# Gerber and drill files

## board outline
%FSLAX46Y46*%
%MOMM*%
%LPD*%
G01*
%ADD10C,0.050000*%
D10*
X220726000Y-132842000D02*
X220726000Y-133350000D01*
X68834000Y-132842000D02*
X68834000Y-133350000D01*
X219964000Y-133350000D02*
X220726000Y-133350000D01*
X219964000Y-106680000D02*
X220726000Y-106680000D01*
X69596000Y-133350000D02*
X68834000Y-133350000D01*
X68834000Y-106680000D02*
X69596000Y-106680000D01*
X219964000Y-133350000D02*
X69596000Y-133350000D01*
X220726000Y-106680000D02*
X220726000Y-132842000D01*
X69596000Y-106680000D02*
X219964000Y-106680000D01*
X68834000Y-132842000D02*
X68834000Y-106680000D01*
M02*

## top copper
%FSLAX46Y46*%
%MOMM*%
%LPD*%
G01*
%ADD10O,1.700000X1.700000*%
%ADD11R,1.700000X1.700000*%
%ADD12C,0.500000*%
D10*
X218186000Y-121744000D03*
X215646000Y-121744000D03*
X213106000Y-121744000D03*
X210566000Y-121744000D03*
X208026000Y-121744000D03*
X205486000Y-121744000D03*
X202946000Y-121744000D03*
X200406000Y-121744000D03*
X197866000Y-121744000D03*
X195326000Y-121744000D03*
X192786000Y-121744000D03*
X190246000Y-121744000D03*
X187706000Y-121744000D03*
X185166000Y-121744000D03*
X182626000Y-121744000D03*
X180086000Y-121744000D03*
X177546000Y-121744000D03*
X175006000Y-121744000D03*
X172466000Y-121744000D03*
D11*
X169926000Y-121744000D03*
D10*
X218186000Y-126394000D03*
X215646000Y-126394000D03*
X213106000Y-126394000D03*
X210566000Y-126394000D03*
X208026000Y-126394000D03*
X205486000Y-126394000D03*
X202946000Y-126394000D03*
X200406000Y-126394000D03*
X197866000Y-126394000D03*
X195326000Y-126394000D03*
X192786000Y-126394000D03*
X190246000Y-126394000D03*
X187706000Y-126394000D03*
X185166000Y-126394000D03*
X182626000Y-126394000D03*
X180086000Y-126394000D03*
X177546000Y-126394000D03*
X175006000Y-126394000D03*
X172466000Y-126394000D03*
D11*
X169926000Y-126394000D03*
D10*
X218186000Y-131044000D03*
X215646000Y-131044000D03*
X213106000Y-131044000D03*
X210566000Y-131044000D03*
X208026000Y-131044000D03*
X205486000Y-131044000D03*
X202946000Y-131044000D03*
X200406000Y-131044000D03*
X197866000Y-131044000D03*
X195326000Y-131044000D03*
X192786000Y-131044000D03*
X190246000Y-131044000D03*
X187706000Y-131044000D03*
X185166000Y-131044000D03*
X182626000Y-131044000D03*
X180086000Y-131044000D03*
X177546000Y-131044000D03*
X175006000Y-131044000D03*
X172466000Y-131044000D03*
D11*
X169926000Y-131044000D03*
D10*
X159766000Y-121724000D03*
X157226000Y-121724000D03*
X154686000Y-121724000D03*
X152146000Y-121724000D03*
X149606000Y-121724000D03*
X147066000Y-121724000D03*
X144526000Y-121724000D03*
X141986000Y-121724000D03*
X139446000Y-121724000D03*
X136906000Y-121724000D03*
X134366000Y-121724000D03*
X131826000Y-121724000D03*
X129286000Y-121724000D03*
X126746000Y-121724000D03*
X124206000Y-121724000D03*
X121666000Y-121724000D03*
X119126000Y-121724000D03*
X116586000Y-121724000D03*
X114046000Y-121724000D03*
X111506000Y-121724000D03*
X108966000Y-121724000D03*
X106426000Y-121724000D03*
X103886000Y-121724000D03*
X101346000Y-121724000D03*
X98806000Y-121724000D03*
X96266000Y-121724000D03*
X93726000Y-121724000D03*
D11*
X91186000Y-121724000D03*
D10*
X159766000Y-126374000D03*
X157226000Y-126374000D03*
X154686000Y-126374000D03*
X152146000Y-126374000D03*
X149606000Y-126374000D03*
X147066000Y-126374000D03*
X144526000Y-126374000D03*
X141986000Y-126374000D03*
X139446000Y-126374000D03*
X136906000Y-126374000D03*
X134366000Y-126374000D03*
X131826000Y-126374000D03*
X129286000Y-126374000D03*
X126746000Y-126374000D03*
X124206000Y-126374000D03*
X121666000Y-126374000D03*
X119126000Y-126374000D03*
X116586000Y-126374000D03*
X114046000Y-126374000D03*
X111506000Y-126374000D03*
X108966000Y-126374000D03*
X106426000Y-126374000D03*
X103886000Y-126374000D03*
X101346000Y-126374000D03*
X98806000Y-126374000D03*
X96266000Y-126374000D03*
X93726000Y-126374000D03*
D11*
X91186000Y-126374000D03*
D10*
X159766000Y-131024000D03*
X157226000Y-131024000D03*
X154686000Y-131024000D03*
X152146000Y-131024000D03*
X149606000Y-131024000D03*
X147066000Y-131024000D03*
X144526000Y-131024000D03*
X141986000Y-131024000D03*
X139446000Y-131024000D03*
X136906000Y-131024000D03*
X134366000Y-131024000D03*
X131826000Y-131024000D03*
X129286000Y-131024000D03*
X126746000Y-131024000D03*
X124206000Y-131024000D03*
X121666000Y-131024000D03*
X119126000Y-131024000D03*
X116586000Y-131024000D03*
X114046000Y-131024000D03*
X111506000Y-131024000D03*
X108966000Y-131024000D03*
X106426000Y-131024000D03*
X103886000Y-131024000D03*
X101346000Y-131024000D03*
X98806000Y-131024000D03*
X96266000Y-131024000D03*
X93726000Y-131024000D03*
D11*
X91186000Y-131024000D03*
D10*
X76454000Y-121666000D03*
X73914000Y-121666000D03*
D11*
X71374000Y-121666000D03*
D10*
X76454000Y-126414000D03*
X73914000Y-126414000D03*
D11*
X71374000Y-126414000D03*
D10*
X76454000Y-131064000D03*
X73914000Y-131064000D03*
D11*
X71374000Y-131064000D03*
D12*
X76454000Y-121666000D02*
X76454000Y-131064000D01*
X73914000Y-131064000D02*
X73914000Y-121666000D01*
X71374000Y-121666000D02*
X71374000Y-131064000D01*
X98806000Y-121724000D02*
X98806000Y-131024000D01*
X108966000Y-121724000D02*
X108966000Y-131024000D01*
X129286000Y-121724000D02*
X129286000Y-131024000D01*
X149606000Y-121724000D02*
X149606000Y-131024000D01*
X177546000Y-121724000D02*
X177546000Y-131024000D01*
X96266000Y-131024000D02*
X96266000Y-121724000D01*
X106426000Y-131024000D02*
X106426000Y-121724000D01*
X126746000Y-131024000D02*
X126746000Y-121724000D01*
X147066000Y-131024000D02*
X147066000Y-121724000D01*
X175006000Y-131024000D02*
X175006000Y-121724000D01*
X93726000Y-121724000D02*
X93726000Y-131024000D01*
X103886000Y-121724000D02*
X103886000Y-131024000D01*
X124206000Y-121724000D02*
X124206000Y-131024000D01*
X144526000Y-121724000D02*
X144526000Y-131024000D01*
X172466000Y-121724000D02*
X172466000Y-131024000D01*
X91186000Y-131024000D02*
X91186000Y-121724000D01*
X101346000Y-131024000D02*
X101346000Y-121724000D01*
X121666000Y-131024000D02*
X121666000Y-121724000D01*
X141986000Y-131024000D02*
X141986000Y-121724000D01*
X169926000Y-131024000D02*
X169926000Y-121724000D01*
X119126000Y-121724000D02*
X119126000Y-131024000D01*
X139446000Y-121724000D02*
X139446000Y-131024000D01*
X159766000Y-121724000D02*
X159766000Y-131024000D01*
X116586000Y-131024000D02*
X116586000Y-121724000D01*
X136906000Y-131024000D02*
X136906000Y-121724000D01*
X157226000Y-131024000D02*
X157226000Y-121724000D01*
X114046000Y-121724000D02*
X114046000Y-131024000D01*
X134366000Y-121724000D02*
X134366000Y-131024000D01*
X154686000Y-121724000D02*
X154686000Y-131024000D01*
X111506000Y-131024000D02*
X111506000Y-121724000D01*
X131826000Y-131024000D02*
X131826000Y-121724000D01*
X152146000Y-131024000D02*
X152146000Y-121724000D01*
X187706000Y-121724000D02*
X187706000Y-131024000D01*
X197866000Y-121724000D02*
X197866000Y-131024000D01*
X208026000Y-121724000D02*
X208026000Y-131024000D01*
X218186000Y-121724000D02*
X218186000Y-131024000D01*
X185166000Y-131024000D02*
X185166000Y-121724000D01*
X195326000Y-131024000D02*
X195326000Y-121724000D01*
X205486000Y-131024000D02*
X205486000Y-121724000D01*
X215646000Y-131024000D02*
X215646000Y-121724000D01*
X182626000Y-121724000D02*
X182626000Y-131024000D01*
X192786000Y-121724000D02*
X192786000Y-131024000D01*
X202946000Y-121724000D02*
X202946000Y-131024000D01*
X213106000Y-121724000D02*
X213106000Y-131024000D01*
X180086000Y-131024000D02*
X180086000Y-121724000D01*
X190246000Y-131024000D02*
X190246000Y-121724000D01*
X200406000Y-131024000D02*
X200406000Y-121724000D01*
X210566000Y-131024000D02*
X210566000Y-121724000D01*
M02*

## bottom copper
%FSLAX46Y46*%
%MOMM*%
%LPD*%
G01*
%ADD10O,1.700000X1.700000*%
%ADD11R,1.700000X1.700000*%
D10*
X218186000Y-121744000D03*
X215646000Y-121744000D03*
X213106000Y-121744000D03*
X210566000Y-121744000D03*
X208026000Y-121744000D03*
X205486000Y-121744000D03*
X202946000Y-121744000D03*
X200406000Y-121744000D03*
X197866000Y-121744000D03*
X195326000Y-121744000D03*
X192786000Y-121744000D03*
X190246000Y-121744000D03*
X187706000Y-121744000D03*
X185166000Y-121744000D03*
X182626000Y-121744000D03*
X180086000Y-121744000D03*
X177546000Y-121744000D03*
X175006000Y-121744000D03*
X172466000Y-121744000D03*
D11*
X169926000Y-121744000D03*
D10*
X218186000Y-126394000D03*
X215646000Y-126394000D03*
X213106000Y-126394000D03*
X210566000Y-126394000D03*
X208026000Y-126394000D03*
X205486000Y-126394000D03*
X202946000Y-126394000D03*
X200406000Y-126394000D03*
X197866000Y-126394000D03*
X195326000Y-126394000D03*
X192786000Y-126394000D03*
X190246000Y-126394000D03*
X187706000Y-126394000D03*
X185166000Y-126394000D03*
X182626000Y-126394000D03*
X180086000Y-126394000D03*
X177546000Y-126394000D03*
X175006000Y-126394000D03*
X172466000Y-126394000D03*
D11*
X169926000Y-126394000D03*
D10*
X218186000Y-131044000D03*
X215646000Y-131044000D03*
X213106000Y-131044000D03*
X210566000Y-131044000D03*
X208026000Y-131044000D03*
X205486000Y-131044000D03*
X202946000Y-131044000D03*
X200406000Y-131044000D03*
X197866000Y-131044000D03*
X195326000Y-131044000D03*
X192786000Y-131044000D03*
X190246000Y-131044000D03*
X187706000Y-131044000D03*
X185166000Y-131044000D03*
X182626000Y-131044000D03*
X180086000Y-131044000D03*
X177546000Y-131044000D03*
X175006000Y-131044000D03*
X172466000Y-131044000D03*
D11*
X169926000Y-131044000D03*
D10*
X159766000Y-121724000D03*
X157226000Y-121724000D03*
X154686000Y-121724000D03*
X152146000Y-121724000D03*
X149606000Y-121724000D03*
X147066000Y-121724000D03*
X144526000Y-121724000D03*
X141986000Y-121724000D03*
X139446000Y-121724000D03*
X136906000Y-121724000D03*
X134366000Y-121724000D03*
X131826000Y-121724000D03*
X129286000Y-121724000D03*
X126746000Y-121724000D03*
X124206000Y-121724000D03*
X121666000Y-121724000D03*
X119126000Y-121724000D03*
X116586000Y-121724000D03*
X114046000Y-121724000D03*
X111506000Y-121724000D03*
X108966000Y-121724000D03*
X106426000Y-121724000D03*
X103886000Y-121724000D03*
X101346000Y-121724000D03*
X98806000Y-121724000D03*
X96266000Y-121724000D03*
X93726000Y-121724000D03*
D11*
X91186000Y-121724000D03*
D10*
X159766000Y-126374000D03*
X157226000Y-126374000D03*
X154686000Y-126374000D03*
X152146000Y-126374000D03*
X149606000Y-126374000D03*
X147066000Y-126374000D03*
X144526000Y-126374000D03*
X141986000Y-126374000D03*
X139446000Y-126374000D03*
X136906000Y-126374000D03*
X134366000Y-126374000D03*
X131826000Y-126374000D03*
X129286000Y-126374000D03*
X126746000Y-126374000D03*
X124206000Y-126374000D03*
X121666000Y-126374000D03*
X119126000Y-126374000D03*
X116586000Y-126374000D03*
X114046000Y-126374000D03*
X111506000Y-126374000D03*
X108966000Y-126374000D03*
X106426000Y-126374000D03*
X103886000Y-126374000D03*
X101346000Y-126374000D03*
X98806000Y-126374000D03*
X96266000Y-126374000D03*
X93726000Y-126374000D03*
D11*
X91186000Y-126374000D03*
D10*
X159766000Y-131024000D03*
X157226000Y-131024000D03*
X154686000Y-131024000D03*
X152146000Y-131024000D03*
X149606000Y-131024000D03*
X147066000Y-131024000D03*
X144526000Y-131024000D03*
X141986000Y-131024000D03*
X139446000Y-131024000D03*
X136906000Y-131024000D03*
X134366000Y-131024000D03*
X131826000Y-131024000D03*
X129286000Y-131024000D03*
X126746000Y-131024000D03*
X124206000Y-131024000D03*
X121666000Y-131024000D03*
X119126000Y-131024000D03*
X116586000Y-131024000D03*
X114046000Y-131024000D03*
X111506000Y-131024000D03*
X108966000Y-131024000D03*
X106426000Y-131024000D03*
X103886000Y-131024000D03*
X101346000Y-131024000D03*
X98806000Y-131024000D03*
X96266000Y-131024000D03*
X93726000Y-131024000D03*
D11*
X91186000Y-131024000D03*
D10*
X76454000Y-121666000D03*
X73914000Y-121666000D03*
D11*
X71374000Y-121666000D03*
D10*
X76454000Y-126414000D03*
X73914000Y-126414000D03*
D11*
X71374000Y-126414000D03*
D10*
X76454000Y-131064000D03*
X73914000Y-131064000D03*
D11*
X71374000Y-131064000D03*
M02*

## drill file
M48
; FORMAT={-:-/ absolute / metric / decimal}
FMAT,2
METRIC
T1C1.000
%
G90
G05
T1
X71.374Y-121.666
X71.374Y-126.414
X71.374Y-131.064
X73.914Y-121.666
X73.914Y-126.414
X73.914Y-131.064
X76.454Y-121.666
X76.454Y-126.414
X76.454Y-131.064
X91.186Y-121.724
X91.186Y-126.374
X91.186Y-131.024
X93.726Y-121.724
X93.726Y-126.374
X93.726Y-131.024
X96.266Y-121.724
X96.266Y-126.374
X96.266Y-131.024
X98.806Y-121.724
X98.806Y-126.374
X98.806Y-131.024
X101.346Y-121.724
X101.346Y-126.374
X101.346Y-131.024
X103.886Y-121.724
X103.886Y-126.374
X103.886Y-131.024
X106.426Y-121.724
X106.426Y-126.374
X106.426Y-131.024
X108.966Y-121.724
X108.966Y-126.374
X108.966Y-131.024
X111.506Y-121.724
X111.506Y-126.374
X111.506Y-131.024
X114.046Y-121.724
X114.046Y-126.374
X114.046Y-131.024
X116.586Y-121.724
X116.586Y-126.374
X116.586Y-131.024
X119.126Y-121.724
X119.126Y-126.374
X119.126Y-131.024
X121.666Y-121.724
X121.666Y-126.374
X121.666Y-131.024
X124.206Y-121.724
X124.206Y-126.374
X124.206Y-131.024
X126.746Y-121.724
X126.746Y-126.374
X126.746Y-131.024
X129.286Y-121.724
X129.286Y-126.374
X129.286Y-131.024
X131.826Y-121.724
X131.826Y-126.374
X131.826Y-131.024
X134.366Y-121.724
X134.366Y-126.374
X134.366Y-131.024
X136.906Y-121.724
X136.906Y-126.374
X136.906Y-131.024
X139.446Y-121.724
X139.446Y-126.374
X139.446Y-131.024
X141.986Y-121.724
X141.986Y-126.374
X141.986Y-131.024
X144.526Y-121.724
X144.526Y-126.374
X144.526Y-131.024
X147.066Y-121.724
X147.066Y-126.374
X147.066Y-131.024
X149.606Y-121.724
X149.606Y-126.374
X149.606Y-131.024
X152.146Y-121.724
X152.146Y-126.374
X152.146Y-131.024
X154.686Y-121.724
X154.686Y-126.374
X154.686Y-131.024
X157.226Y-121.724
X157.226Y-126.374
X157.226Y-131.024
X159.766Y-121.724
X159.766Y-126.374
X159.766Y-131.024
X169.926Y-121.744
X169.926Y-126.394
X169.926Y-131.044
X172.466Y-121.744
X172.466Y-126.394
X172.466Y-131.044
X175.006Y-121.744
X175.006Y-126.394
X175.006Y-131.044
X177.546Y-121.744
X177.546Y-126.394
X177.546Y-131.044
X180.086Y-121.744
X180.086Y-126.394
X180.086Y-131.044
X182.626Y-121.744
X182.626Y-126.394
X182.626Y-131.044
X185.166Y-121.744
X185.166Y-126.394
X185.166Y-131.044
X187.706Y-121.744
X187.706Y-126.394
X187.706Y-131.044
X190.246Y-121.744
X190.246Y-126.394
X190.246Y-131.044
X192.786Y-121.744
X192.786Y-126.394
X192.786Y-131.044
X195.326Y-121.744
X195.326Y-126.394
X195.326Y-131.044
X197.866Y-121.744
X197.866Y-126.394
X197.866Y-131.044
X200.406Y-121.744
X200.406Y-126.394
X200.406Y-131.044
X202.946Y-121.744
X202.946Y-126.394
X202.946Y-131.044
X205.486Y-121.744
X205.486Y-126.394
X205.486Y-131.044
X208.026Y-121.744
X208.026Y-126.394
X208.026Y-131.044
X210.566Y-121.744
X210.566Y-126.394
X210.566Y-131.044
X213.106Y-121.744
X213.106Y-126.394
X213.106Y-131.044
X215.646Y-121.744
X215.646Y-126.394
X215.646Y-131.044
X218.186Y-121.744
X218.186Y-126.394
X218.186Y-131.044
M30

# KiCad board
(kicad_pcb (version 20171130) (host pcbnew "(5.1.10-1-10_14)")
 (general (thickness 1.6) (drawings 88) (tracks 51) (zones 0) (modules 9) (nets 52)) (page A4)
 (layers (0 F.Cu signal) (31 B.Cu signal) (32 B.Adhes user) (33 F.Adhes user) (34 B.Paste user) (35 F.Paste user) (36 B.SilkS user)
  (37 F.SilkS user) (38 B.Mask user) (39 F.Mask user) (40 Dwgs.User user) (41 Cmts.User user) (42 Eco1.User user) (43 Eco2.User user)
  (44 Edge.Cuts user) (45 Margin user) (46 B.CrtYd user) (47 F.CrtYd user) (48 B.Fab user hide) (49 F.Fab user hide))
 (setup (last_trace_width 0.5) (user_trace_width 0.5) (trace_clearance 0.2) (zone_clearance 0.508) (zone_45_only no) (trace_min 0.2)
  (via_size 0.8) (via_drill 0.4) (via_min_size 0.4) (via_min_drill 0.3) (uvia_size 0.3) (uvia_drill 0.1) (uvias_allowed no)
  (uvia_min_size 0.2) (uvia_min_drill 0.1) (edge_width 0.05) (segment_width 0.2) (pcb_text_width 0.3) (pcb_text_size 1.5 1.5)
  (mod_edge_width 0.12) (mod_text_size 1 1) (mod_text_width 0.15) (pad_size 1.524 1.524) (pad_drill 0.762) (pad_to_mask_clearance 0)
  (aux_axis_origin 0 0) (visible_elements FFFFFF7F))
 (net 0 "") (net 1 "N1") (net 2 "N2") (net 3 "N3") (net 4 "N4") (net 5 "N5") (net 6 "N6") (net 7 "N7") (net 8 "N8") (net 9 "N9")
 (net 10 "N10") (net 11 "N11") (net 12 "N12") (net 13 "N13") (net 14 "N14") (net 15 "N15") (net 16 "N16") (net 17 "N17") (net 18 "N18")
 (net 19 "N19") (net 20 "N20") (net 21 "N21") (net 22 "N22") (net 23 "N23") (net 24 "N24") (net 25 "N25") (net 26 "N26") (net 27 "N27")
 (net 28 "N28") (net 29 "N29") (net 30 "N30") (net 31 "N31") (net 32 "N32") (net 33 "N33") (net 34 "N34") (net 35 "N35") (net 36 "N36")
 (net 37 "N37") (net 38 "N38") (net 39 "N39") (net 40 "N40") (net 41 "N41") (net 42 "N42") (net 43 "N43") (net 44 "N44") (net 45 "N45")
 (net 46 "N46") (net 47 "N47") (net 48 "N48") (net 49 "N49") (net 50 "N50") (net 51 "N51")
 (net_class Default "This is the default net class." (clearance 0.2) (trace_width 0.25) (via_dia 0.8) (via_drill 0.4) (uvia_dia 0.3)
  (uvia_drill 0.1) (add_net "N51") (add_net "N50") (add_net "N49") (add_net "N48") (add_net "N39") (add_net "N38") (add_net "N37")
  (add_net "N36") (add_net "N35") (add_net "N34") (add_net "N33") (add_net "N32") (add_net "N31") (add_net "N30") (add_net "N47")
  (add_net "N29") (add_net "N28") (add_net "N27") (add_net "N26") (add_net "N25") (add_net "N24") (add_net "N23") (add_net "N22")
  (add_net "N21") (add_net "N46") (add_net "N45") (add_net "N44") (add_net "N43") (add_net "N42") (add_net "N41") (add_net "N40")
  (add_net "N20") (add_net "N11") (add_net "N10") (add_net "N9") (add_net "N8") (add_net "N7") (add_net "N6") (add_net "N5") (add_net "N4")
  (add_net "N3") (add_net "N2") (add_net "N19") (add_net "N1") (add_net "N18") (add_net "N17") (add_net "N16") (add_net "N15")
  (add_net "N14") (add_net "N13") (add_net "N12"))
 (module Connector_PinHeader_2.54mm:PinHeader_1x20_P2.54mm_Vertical (layer F.Cu) (at 169.926 121.744 90)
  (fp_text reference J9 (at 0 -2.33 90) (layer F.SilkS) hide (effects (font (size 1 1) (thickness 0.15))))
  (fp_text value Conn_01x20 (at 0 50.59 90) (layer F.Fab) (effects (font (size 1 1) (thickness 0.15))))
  (pad 20 thru_hole oval (at 0 48.26 90) (size 1.7 1.7) (drill 1) (layers *.Cu *.Mask) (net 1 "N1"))
  (pad 19 thru_hole oval (at 0 45.72 90) (size 1.7 1.7) (drill 1) (layers *.Cu *.Mask) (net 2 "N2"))
  (pad 18 thru_hole oval (at 0 43.18 90) (size 1.7 1.7) (drill 1) (layers *.Cu *.Mask) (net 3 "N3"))
  (pad 17 thru_hole oval (at 0 40.64 90) (size 1.7 1.7) (drill 1) (layers *.Cu *.Mask) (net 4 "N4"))
  (pad 16 thru_hole oval (at 0 38.1 90) (size 1.7 1.7) (drill 1) (layers *.Cu *.Mask) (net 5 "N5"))
  (pad 15 thru_hole oval (at 0 35.56 90) (size 1.7 1.7) (drill 1) (layers *.Cu *.Mask) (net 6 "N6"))
  (pad 14 thru_hole oval (at 0 33.02 90) (size 1.7 1.7) (drill 1) (layers *.Cu *.Mask) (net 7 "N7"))
  (pad 13 thru_hole oval (at 0 30.48 90) (size 1.7 1.7) (drill 1) (layers *.Cu *.Mask) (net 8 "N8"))
  (pad 12 thru_hole oval (at 0 27.94 90) (size 1.7 1.7) (drill 1) (layers *.Cu *.Mask) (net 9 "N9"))
  (pad 11 thru_hole oval (at 0 25.4 90) (size 1.7 1.7) (drill 1) (layers *.Cu *.Mask) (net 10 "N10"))
  (pad 10 thru_hole oval (at 0 22.86 90) (size 1.7 1.7) (drill 1) (layers *.Cu *.Mask) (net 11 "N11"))
  (pad 9 thru_hole oval (at 0 20.32 90) (size 1.7 1.7) (drill 1) (layers *.Cu *.Mask) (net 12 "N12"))
  (pad 8 thru_hole oval (at 0 17.78 90) (size 1.7 1.7) (drill 1) (layers *.Cu *.Mask) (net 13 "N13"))
  (pad 7 thru_hole oval (at 0 15.24 90) (size 1.7 1.7) (drill 1) (layers *.Cu *.Mask) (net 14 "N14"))
  (pad 6 thru_hole oval (at 0 12.7 90) (size 1.7 1.7) (drill 1) (layers *.Cu *.Mask) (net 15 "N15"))
  (pad 5 thru_hole oval (at 0 10.16 90) (size 1.7 1.7) (drill 1) (layers *.Cu *.Mask) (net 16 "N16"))
  (pad 4 thru_hole oval (at 0 7.62 90) (size 1.7 1.7) (drill 1) (layers *.Cu *.Mask) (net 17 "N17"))
  (pad 3 thru_hole oval (at 0 5.08 90) (size 1.7 1.7) (drill 1) (layers *.Cu *.Mask) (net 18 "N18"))
  (pad 2 thru_hole oval (at 0 2.54 90) (size 1.7 1.7) (drill 1) (layers *.Cu *.Mask) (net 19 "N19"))
  (pad 1 thru_hole rect (at 0 0 90) (size 1.7 1.7) (drill 1) (layers *.Cu *.Mask) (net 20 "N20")))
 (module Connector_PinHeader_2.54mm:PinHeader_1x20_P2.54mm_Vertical (layer F.Cu) (at 169.926 126.394 90)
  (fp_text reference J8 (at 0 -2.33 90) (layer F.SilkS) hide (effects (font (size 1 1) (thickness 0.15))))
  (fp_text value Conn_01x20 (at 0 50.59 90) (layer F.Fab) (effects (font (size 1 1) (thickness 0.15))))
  (pad 20 thru_hole oval (at 0 48.26 90) (size 1.7 1.7) (drill 1) (layers *.Cu *.Mask) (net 1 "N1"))
  (pad 19 thru_hole oval (at 0 45.72 90) (size 1.7 1.7) (drill 1) (layers *.Cu *.Mask) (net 2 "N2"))
  (pad 18 thru_hole oval (at 0 43.18 90) (size 1.7 1.7) (drill 1) (layers *.Cu *.Mask) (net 3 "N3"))
  (pad 17 thru_hole oval (at 0 40.64 90) (size 1.7 1.7) (drill 1) (layers *.Cu *.Mask) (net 4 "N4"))
  (pad 16 thru_hole oval (at 0 38.1 90) (size 1.7 1.7) (drill 1) (layers *.Cu *.Mask) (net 5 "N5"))
  (pad 15 thru_hole oval (at 0 35.56 90) (size 1.7 1.7) (drill 1) (layers *.Cu *.Mask) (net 6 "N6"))
  (pad 14 thru_hole oval (at 0 33.02 90) (size 1.7 1.7) (drill 1) (layers *.Cu *.Mask) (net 7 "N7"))
  (pad 13 thru_hole oval (at 0 30.48 90) (size 1.7 1.7) (drill 1) (layers *.Cu *.Mask) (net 8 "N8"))
  (pad 12 thru_hole oval (at 0 27.94 90) (size 1.7 1.7) (drill 1) (layers *.Cu *.Mask) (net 9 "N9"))
  (pad 11 thru_hole oval (at 0 25.4 90) (size 1.7 1.7) (drill 1) (layers *.Cu *.Mask) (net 10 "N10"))
  (pad 10 thru_hole oval (at 0 22.86 90) (size 1.7 1.7) (drill 1) (layers *.Cu *.Mask) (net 11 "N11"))
  (pad 9 thru_hole oval (at 0 20.32 90) (size 1.7 1.7) (drill 1) (layers *.Cu *.Mask) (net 12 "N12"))
  (pad 8 thru_hole oval (at 0 17.78 90) (size 1.7 1.7) (drill 1) (layers *.Cu *.Mask) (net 13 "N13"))
  (pad 7 thru_hole oval (at 0 15.24 90) (size 1.7 1.7) (drill 1) (layers *.Cu *.Mask) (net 14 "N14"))
  (pad 6 thru_hole oval (at 0 12.7 90) (size 1.7 1.7) (drill 1) (layers *.Cu *.Mask) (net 15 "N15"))
  (pad 5 thru_hole oval (at 0 10.16 90) (size 1.7 1.7) (drill 1) (layers *.Cu *.Mask) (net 16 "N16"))
  (pad 4 thru_hole oval (at 0 7.62 90) (size 1.7 1.7) (drill 1) (layers *.Cu *.Mask) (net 17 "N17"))
  (pad 3 thru_hole oval (at 0 5.08 90) (size 1.7 1.7) (drill 1) (layers *.Cu *.Mask) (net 18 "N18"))
  (pad 2 thru_hole oval (at 0 2.54 90) (size 1.7 1.7) (drill 1) (layers *.Cu *.Mask) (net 19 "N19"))
  (pad 1 thru_hole rect (at 0 0 90) (size 1.7 1.7) (drill 1) (layers *.Cu *.Mask) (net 20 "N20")))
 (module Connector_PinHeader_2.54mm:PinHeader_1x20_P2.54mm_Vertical (layer F.Cu) (at 169.926 131.044 90)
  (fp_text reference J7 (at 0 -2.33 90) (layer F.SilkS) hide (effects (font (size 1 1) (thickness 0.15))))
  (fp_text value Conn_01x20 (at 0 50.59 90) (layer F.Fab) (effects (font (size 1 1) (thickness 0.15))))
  (pad 20 thru_hole oval (at 0 48.26 90) (size 1.7 1.7) (drill 1) (layers *.Cu *.Mask) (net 1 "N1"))
  (pad 19 thru_hole oval (at 0 45.72 90) (size 1.7 1.7) (drill 1) (layers *.Cu *.Mask) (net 2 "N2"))
  (pad 18 thru_hole oval (at 0 43.18 90) (size 1.7 1.7) (drill 1) (layers *.Cu *.Mask) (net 3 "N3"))
  (pad 17 thru_hole oval (at 0 40.64 90) (size 1.7 1.7) (drill 1) (layers *.Cu *.Mask) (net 4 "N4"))
  (pad 16 thru_hole oval (at 0 38.1 90) (size 1.7 1.7) (drill 1) (layers *.Cu *.Mask) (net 5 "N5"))
  (pad 15 thru_hole oval (at 0 35.56 90) (size 1.7 1.7) (drill 1) (layers *.Cu *.Mask) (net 6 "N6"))
  (pad 14 thru_hole oval (at 0 33.02 90) (size 1.7 1.7) (drill 1) (layers *.Cu *.Mask) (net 7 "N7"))
  (pad 13 thru_hole oval (at 0 30.48 90) (size 1.7 1.7) (drill 1) (layers *.Cu *.Mask) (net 8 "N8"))
  (pad 12 thru_hole oval (at 0 27.94 90) (size 1.7 1.7) (drill 1) (layers *.Cu *.Mask) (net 9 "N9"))
  (pad 11 thru_hole oval (at 0 25.4 90) (size 1.7 1.7) (drill 1) (layers *.Cu *.Mask) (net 10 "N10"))
  (pad 10 thru_hole oval (at 0 22.86 90) (size 1.7 1.7) (drill 1) (layers *.Cu *.Mask) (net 11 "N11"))
  (pad 9 thru_hole oval (at 0 20.32 90) (size 1.7 1.7) (drill 1) (layers *.Cu *.Mask) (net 12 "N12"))
  (pad 8 thru_hole oval (at 0 17.78 90) (size 1.7 1.7) (drill 1) (layers *.Cu *.Mask) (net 13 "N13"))
  (pad 7 thru_hole oval (at 0 15.24 90) (size 1.7 1.7) (drill 1) (layers *.Cu *.Mask) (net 14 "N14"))
  (pad 6 thru_hole oval (at 0 12.7 90) (size 1.7 1.7) (drill 1) (layers *.Cu *.Mask) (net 15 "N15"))
  (pad 5 thru_hole oval (at 0 10.16 90) (size 1.7 1.7) (drill 1) (layers *.Cu *.Mask) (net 16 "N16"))
  (pad 4 thru_hole oval (at 0 7.62 90) (size 1.7 1.7) (drill 1) (layers *.Cu *.Mask) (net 17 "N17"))
  (pad 3 thru_hole oval (at 0 5.08 90) (size 1.7 1.7) (drill 1) (layers *.Cu *.Mask) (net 18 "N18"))
  (pad 2 thru_hole oval (at 0 2.54 90) (size 1.7 1.7) (drill 1) (layers *.Cu *.Mask) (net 19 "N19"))
  (pad 1 thru_hole rect (at 0 0 90) (size 1.7 1.7) (drill 1) (layers *.Cu *.Mask) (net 20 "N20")))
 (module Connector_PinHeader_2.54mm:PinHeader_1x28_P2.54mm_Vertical (layer F.Cu) (at 91.186 121.724 90)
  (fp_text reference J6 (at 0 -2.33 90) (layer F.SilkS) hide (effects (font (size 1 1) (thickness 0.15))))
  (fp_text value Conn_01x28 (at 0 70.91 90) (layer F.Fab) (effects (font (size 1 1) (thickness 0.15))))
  (pad 28 thru_hole oval (at 0 68.58 90) (size 1.7 1.7) (drill 1) (layers *.Cu *.Mask) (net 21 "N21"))
  (pad 27 thru_hole oval (at 0 66.04 90) (size 1.7 1.7) (drill 1) (layers *.Cu *.Mask) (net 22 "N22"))
  (pad 26 thru_hole oval (at 0 63.5 90) (size 1.7 1.7) (drill 1) (layers *.Cu *.Mask) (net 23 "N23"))
  (pad 25 thru_hole oval (at 0 60.96 90) (size 1.7 1.7) (drill 1) (layers *.Cu *.Mask) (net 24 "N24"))
  (pad 24 thru_hole oval (at 0 58.42 90) (size 1.7 1.7) (drill 1) (layers *.Cu *.Mask) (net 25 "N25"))
  (pad 23 thru_hole oval (at 0 55.88 90) (size 1.7 1.7) (drill 1) (layers *.Cu *.Mask) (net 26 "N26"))
  (pad 22 thru_hole oval (at 0 53.34 90) (size 1.7 1.7) (drill 1) (layers *.Cu *.Mask) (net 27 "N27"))
  (pad 21 thru_hole oval (at 0 50.8 90) (size 1.7 1.7) (drill 1) (layers *.Cu *.Mask) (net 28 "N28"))
  (pad 20 thru_hole oval (at 0 48.26 90) (size 1.7 1.7) (drill 1) (layers *.Cu *.Mask) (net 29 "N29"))
  (pad 19 thru_hole oval (at 0 45.72 90) (size 1.7 1.7) (drill 1) (layers *.Cu *.Mask) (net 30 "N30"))
  (pad 18 thru_hole oval (at 0 43.18 90) (size 1.7 1.7) (drill 1) (layers *.Cu *.Mask) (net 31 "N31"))
  (pad 17 thru_hole oval (at 0 40.64 90) (size 1.7 1.7) (drill 1) (layers *.Cu *.Mask) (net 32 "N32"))
  (pad 16 thru_hole oval (at 0 38.1 90) (size 1.7 1.7) (drill 1) (layers *.Cu *.Mask) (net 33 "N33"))
  (pad 15 thru_hole oval (at 0 35.56 90) (size 1.7 1.7) (drill 1) (layers *.Cu *.Mask) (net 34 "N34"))
  (pad 14 thru_hole oval (at 0 33.02 90) (size 1.7 1.7) (drill 1) (layers *.Cu *.Mask) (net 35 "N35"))
  (pad 13 thru_hole oval (at 0 30.48 90) (size 1.7 1.7) (drill 1) (layers *.Cu *.Mask) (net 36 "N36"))
  (pad 12 thru_hole oval (at 0 27.94 90) (size 1.7 1.7) (drill 1) (layers *.Cu *.Mask) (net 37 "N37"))
  (pad 11 thru_hole oval (at 0 25.4 90) (size 1.7 1.7) (drill 1) (layers *.Cu *.Mask) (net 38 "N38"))
  (pad 10 thru_hole oval (at 0 22.86 90) (size 1.7 1.7) (drill 1) (layers *.Cu *.Mask) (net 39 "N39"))
  (pad 9 thru_hole oval (at 0 20.32 90) (size 1.7 1.7) (drill 1) (layers *.Cu *.Mask) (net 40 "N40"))
  (pad 8 thru_hole oval (at 0 17.78 90) (size 1.7 1.7) (drill 1) (layers *.Cu *.Mask) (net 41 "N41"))
  (pad 7 thru_hole oval (at 0 15.24 90) (size 1.7 1.7) (drill 1) (layers *.Cu *.Mask) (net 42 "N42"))
  (pad 6 thru_hole oval (at 0 12.7 90) (size 1.7 1.7) (drill 1) (layers *.Cu *.Mask) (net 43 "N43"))
  (pad 5 thru_hole oval (at 0 10.16 90) (size 1.7 1.7) (drill 1) (layers *.Cu *.Mask) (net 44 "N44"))
  (pad 4 thru_hole oval (at 0 7.62 90) (size 1.7 1.7) (drill 1) (layers *.Cu *.Mask) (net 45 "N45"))
  (pad 3 thru_hole oval (at 0 5.08 90) (size 1.7 1.7) (drill 1) (layers *.Cu *.Mask) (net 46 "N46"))
  (pad 2 thru_hole oval (at 0 2.54 90) (size 1.7 1.7) (drill 1) (layers *.Cu *.Mask) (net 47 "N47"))
  (pad 1 thru_hole rect (at 0 0 90) (size 1.7 1.7) (drill 1) (layers *.Cu *.Mask) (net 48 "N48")))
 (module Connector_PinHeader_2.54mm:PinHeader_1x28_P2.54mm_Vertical (layer F.Cu) (at 91.186 126.374 90)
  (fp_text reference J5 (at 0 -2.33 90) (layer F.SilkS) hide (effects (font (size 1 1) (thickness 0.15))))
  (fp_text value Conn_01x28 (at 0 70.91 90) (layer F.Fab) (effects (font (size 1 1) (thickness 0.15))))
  (pad 28 thru_hole oval (at 0 68.58 90) (size 1.7 1.7) (drill 1) (layers *.Cu *.Mask) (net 21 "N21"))
  (pad 27 thru_hole oval (at 0 66.04 90) (size 1.7 1.7) (drill 1) (layers *.Cu *.Mask) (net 22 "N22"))
  (pad 26 thru_hole oval (at 0 63.5 90) (size 1.7 1.7) (drill 1) (layers *.Cu *.Mask) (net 23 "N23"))
  (pad 25 thru_hole oval (at 0 60.96 90) (size 1.7 1.7) (drill 1) (layers *.Cu *.Mask) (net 24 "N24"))
  (pad 24 thru_hole oval (at 0 58.42 90) (size 1.7 1.7) (drill 1) (layers *.Cu *.Mask) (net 25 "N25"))
  (pad 23 thru_hole oval (at 0 55.88 90) (size 1.7 1.7) (drill 1) (layers *.Cu *.Mask) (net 26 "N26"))
  (pad 22 thru_hole oval (at 0 53.34 90) (size 1.7 1.7) (drill 1) (layers *.Cu *.Mask) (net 27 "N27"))
  (pad 21 thru_hole oval (at 0 50.8 90) (size 1.7 1.7) (drill 1) (layers *.Cu *.Mask) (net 28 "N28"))
  (pad 20 thru_hole oval (at 0 48.26 90) (size 1.7 1.7) (drill 1) (layers *.Cu *.Mask) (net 29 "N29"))
  (pad 19 thru_hole oval (at 0 45.72 90) (size 1.7 1.7) (drill 1) (layers *.Cu *.Mask) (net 30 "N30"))
  (pad 18 thru_hole oval (at 0 43.18 90) (size 1.7 1.7) (drill 1) (layers *.Cu *.Mask) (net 31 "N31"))
  (pad 17 thru_hole oval (at 0 40.64 90) (size 1.7 1.7) (drill 1) (layers *.Cu *.Mask) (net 32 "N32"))
  (pad 16 thru_hole oval (at 0 38.1 90) (size 1.7 1.7) (drill 1) (layers *.Cu *.Mask) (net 33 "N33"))
  (pad 15 thru_hole oval (at 0 35.56 90) (size 1.7 1.7) (drill 1) (layers *.Cu *.Mask) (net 34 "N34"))
  (pad 14 thru_hole oval (at 0 33.02 90) (size 1.7 1.7) (drill 1) (layers *.Cu *.Mask) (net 35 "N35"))
  (pad 13 thru_hole oval (at 0 30.48 90) (size 1.7 1.7) (drill 1) (layers *.Cu *.Mask) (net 36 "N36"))
  (pad 12 thru_hole oval (at 0 27.94 90) (size 1.7 1.7) (drill 1) (layers *.Cu *.Mask) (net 37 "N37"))
  (pad 11 thru_hole oval (at 0 25.4 90) (size 1.7 1.7) (drill 1) (layers *.Cu *.Mask) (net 38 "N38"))
  (pad 10 thru_hole oval (at 0 22.86 90) (size 1.7 1.7) (drill 1) (layers *.Cu *.Mask) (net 39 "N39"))
  (pad 9 thru_hole oval (at 0 20.32 90) (size 1.7 1.7) (drill 1) (layers *.Cu *.Mask) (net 40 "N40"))
  (pad 8 thru_hole oval (at 0 17.78 90) (size 1.7 1.7) (drill 1) (layers *.Cu *.Mask) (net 41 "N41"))
  (pad 7 thru_hole oval (at 0 15.24 90) (size 1.7 1.7) (drill 1) (layers *.Cu *.Mask) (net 42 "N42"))
  (pad 6 thru_hole oval (at 0 12.7 90) (size 1.7 1.7) (drill 1) (layers *.Cu *.Mask) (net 43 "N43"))
  (pad 5 thru_hole oval (at 0 10.16 90) (size 1.7 1.7) (drill 1) (layers *.Cu *.Mask) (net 44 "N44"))
  (pad 4 thru_hole oval (at 0 7.62 90) (size 1.7 1.7) (drill 1) (layers *.Cu *.Mask) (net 45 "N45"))
  (pad 3 thru_hole oval (at 0 5.08 90) (size 1.7 1.7) (drill 1) (layers *.Cu *.Mask) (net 46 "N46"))
  (pad 2 thru_hole oval (at 0 2.54 90) (size 1.7 1.7) (drill 1) (layers *.Cu *.Mask) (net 47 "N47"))
  (pad 1 thru_hole rect (at 0 0 90) (size 1.7 1.7) (drill 1) (layers *.Cu *.Mask) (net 48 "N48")))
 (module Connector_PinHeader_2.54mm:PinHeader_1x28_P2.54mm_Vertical (layer F.Cu) (at 91.186 131.024 90)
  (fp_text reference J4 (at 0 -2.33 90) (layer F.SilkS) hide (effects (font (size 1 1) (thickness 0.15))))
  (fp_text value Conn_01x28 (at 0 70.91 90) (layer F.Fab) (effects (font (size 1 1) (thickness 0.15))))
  (pad 28 thru_hole oval (at 0 68.58 90) (size 1.7 1.7) (drill 1) (layers *.Cu *.Mask) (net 21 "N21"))
  (pad 27 thru_hole oval (at 0 66.04 90) (size 1.7 1.7) (drill 1) (layers *.Cu *.Mask) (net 22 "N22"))
  (pad 26 thru_hole oval (at 0 63.5 90) (size 1.7 1.7) (drill 1) (layers *.Cu *.Mask) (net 23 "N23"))
  (pad 25 thru_hole oval (at 0 60.96 90) (size 1.7 1.7) (drill 1) (layers *.Cu *.Mask) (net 24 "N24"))
  (pad 24 thru_hole oval (at 0 58.42 90) (size 1.7 1.7) (drill 1) (layers *.Cu *.Mask) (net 25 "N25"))
  (pad 23 thru_hole oval (at 0 55.88 90) (size 1.7 1.7) (drill 1) (layers *.Cu *.Mask) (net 26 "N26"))
  (pad 22 thru_hole oval (at 0 53.34 90) (size 1.7 1.7) (drill 1) (layers *.Cu *.Mask) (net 27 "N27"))
  (pad 21 thru_hole oval (at 0 50.8 90) (size 1.7 1.7) (drill 1) (layers *.Cu *.Mask) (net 28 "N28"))
  (pad 20 thru_hole oval (at 0 48.26 90) (size 1.7 1.7) (drill 1) (layers *.Cu *.Mask) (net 29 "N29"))
  (pad 19 thru_hole oval (at 0 45.72 90) (size 1.7 1.7) (drill 1) (layers *.Cu *.Mask) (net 30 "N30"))
  (pad 18 thru_hole oval (at 0 43.18 90) (size 1.7 1.7) (drill 1) (layers *.Cu *.Mask) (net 31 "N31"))
  (pad 17 thru_hole oval (at 0 40.64 90) (size 1.7 1.7) (drill 1) (layers *.Cu *.Mask) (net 32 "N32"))
  (pad 16 thru_hole oval (at 0 38.1 90) (size 1.7 1.7) (drill 1) (layers *.Cu *.Mask) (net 33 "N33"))
  (pad 15 thru_hole oval (at 0 35.56 90) (size 1.7 1.7) (drill 1) (layers *.Cu *.Mask) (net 34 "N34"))
  (pad 14 thru_hole oval (at 0 33.02 90) (size 1.7 1.7) (drill 1) (layers *.Cu *.Mask) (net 35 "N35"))
  (pad 13 thru_hole oval (at 0 30.48 90) (size 1.7 1.7) (drill 1) (layers *.Cu *.Mask) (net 36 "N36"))
  (pad 12 thru_hole oval (at 0 27.94 90) (size 1.7 1.7) (drill 1) (layers *.Cu *.Mask) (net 37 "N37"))
  (pad 11 thru_hole oval (at 0 25.4 90) (size 1.7 1.7) (drill 1) (layers *.Cu *.Mask) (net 38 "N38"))
  (pad 10 thru_hole oval (at 0 22.86 90) (size 1.7 1.7) (drill 1) (layers *.Cu *.Mask) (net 39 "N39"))
  (pad 9 thru_hole oval (at 0 20.32 90) (size 1.7 1.7) (drill 1) (layers *.Cu *.Mask) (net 40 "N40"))
  (pad 8 thru_hole oval (at 0 17.78 90) (size 1.7 1.7) (drill 1) (layers *.Cu *.Mask) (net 41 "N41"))
  (pad 7 thru_hole oval (at 0 15.24 90) (size 1.7 1.7) (drill 1) (layers *.Cu *.Mask) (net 42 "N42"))
  (pad 6 thru_hole oval (at 0 12.7 90) (size 1.7 1.7) (drill 1) (layers *.Cu *.Mask) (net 43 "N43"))
  (pad 5 thru_hole oval (at 0 10.16 90) (size 1.7 1.7) (drill 1) (layers *.Cu *.Mask) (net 44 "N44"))
  (pad 4 thru_hole oval (at 0 7.62 90) (size 1.7 1.7) (drill 1) (layers *.Cu *.Mask) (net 45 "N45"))
  (pad 3 thru_hole oval (at 0 5.08 90) (size 1.7 1.7) (drill 1) (layers *.Cu *.Mask) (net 46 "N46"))
  (pad 2 thru_hole oval (at 0 2.54 90) (size 1.7 1.7) (drill 1) (layers *.Cu *.Mask) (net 47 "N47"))
  (pad 1 thru_hole rect (at 0 0 90) (size 1.7 1.7) (drill 1) (layers *.Cu *.Mask) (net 48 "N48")))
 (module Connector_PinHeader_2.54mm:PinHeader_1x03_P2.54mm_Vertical (layer F.Cu) (at 71.374 121.666 90)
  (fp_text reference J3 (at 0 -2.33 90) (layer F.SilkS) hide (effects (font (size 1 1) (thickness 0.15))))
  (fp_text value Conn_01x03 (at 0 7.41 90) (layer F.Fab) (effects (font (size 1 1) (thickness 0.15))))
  (pad 3 thru_hole oval (at 0 5.08 90) (size 1.7 1.7) (drill 1) (layers *.Cu *.Mask) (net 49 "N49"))
  (pad 2 thru_hole oval (at 0 2.54 90) (size 1.7 1.7) (drill 1) (layers *.Cu *.Mask) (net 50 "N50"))
  (pad 1 thru_hole rect (at 0 0 90) (size 1.7 1.7) (drill 1) (layers *.Cu *.Mask) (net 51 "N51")))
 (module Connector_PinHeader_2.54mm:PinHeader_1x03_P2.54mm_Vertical (layer F.Cu) (at 71.374 126.414 90)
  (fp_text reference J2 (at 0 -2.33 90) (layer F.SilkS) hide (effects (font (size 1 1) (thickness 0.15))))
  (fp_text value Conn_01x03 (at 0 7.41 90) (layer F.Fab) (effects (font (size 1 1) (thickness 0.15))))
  (pad 3 thru_hole oval (at 0 5.08 90) (size 1.7 1.7) (drill 1) (layers *.Cu *.Mask) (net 49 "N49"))
  (pad 2 thru_hole oval (at 0 2.54 90) (size 1.7 1.7) (drill 1) (layers *.Cu *.Mask) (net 50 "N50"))
  (pad 1 thru_hole rect (at 0 0 90) (size 1.7 1.7) (drill 1) (layers *.Cu *.Mask) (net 51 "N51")))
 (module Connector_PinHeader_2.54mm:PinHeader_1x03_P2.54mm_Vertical (layer F.Cu) (at 71.374 131.064 90)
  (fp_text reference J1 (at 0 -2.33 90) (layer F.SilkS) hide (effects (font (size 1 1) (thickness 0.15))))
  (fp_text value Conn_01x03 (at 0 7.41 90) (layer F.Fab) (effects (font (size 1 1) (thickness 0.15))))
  (pad 3 thru_hole oval (at 0 5.08 90) (size 1.7 1.7) (drill 1) (layers *.Cu *.Mask) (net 49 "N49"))
  (pad 2 thru_hole oval (at 0 2.54 90) (size 1.7 1.7) (drill 1) (layers *.Cu *.Mask) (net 50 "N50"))
  (pad 1 thru_hole rect (at 0 0 90) (size 1.7 1.7) (drill 1) (layers *.Cu *.Mask) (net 51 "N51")))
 (gr_line (start 220.726 132.842) (end 220.726 133.35) (layer Edge.Cuts) (width 0.05))
 (gr_line (start 68.834 132.842) (end 68.834 133.35) (layer Edge.Cuts) (width 0.05))
 (gr_line (start 219.964 133.35) (end 220.726 133.35) (layer Edge.Cuts) (width 0.05))
 (gr_line (start 219.964 106.68) (end 220.726 106.68) (layer Edge.Cuts) (width 0.05))
 (gr_line (start 69.596 133.35) (end 68.834 133.35) (layer Edge.Cuts) (width 0.05))
 (gr_line (start 68.834 106.68) (end 69.596 106.68) (layer Edge.Cuts) (width 0.05))
 (gr_line (start 219.964 133.35) (end 69.596 133.35) (layer Edge.Cuts) (width 0.05))
 (gr_line (start 220.726 106.68) (end 220.726 132.842) (layer Edge.Cuts) (width 0.05))
 (gr_line (start 69.596 106.68) (end 219.964 106.68) (layer Edge.Cuts) (width 0.05))
 (gr_line (start 68.834 132.842) (end 68.834 106.68) (layer Edge.Cuts) (width 0.05))
 (segment (start 76.454 121.666) (end 76.454 131.064) (width 0.5) (layer F.Cu) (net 49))
 (segment (start 73.914 131.064) (end 73.914 121.666) (width 0.5) (layer F.Cu) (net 50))
 (segment (start 71.374 121.666) (end 71.374 131.064) (width 0.5) (layer F.Cu) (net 51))
 (segment (start 98.806 121.724) (end 98.806 131.024) (width 0.5) (layer F.Cu) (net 45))
 (segment (start 108.966 121.724) (end 108.966 131.024) (width 0.5) (layer F.Cu) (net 41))
 (segment (start 129.286 121.724) (end 129.286 131.024) (width 0.5) (layer F.Cu) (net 33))
 (segment (start 149.606 121.724) (end 149.606 131.024) (width 0.5) (layer F.Cu) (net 25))
 (segment (start 177.546 121.724) (end 177.546 131.024) (width 0.5) (layer F.Cu) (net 17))
 (segment (start 96.266 131.024) (end 96.266 121.724) (width 0.5) (layer F.Cu) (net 46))
 (segment (start 106.426 131.024) (end 106.426 121.724) (width 0.5) (layer F.Cu) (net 42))
 (segment (start 126.746 131.024) (end 126.746 121.724) (width 0.5) (layer F.Cu) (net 34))
 (segment (start 147.066 131.024) (end 147.066 121.724) (width 0.5) (layer F.Cu) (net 26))
 (segment (start 175.006 131.024) (end 175.006 121.724) (width 0.5) (layer F.Cu) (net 18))
 (segment (start 93.726 121.724) (end 93.726 131.024) (width 0.5) (layer F.Cu) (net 47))
 (segment (start 103.886 121.724) (end 103.886 131.024) (width 0.5) (layer F.Cu) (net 43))
 (segment (start 124.206 121.724) (end 124.206 131.024) (width 0.5) (layer F.Cu) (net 35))
 (segment (start 144.526 121.724) (end 144.526 131.024) (width 0.5) (layer F.Cu) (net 27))
 (segment (start 172.466 121.724) (end 172.466 131.024) (width 0.5) (layer F.Cu) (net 19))
 (segment (start 91.186 131.024) (end 91.186 121.724) (width 0.5) (layer F.Cu) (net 48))
 (segment (start 101.346 131.024) (end 101.346 121.724) (width 0.5) (layer F.Cu) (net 44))
 (segment (start 121.666 131.024) (end 121.666 121.724) (width 0.5) (layer F.Cu) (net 36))
 (segment (start 141.986 131.024) (end 141.986 121.724) (width 0.5) (layer F.Cu) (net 28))
 (segment (start 169.926 131.024) (end 169.926 121.724) (width 0.5) (layer F.Cu) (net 20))
 (segment (start 119.126 121.724) (end 119.126 131.024) (width 0.5) (layer F.Cu) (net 37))
 (segment (start 139.446 121.724) (end 139.446 131.024) (width 0.5) (layer F.Cu) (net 29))
 (segment (start 159.766 121.724) (end 159.766 131.024) (width 0.5) (layer F.Cu) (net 21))
 (segment (start 116.586 131.024) (end 116.586 121.724) (width 0.5) (layer F.Cu) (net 38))
 (segment (start 136.906 131.024) (end 136.906 121.724) (width 0.5) (layer F.Cu) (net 30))
 (segment (start 157.226 131.024) (end 157.226 121.724) (width 0.5) (layer F.Cu) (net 22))
 (segment (start 114.046 121.724) (end 114.046 131.024) (width 0.5) (layer F.Cu) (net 39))
 (segment (start 134.366 121.724) (end 134.366 131.024) (width 0.5) (layer F.Cu) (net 31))
 (segment (start 154.686 121.724) (end 154.686 131.024) (width 0.5) (layer F.Cu) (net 23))
 (segment (start 111.506 131.024) (end 111.506 121.724) (width 0.5) (layer F.Cu) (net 40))
 (segment (start 131.826 131.024) (end 131.826 121.724) (width 0.5) (layer F.Cu) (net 32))
 (segment (start 152.146 131.024) (end 152.146 121.724) (width 0.5) (layer F.Cu) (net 24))
 (segment (start 187.706 121.724) (end 187.706 131.024) (width 0.5) (layer F.Cu) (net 13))
 (segment (start 197.866 121.724) (end 197.866 131.024) (width 0.5) (layer F.Cu) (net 9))
 (segment (start 208.026 121.724) (end 208.026 131.024) (width 0.5) (layer F.Cu) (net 5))
 (segment (start 218.186 121.724) (end 218.186 131.024) (width 0.5) (layer F.Cu) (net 1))
 (segment (start 185.166 131.024) (end 185.166 121.724) (width 0.5) (layer F.Cu) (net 14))
 (segment (start 195.326 131.024) (end 195.326 121.724) (width 0.5) (layer F.Cu) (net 10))
 (segment (start 205.486 131.024) (end 205.486 121.724) (width 0.5) (layer F.Cu) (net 6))
 (segment (start 215.646 131.024) (end 215.646 121.724) (width 0.5) (layer F.Cu) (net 2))
 (segment (start 182.626 121.724) (end 182.626 131.024) (width 0.5) (layer F.Cu) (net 15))
 (segment (start 192.786 121.724) (end 192.786 131.024) (width 0.5) (layer F.Cu) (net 11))
 (segment (start 202.946 121.724) (end 202.946 131.024) (width 0.5) (layer F.Cu) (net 7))
 (segment (start 213.106 121.724) (end 213.106 131.024) (width 0.5) (layer F.Cu) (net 3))
 (segment (start 180.086 131.024) (end 180.086 121.724) (width 0.5) (layer F.Cu) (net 16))
 (segment (start 190.246 131.024) (end 190.246 121.724) (width 0.5) (layer F.Cu) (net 12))
 (segment (start 200.406 131.024) (end 200.406 121.724) (width 0.5) (layer F.Cu) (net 8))
 (segment (start 210.566 131.024) (end 210.566 121.724) (width 0.5) (layer F.Cu) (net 4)))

